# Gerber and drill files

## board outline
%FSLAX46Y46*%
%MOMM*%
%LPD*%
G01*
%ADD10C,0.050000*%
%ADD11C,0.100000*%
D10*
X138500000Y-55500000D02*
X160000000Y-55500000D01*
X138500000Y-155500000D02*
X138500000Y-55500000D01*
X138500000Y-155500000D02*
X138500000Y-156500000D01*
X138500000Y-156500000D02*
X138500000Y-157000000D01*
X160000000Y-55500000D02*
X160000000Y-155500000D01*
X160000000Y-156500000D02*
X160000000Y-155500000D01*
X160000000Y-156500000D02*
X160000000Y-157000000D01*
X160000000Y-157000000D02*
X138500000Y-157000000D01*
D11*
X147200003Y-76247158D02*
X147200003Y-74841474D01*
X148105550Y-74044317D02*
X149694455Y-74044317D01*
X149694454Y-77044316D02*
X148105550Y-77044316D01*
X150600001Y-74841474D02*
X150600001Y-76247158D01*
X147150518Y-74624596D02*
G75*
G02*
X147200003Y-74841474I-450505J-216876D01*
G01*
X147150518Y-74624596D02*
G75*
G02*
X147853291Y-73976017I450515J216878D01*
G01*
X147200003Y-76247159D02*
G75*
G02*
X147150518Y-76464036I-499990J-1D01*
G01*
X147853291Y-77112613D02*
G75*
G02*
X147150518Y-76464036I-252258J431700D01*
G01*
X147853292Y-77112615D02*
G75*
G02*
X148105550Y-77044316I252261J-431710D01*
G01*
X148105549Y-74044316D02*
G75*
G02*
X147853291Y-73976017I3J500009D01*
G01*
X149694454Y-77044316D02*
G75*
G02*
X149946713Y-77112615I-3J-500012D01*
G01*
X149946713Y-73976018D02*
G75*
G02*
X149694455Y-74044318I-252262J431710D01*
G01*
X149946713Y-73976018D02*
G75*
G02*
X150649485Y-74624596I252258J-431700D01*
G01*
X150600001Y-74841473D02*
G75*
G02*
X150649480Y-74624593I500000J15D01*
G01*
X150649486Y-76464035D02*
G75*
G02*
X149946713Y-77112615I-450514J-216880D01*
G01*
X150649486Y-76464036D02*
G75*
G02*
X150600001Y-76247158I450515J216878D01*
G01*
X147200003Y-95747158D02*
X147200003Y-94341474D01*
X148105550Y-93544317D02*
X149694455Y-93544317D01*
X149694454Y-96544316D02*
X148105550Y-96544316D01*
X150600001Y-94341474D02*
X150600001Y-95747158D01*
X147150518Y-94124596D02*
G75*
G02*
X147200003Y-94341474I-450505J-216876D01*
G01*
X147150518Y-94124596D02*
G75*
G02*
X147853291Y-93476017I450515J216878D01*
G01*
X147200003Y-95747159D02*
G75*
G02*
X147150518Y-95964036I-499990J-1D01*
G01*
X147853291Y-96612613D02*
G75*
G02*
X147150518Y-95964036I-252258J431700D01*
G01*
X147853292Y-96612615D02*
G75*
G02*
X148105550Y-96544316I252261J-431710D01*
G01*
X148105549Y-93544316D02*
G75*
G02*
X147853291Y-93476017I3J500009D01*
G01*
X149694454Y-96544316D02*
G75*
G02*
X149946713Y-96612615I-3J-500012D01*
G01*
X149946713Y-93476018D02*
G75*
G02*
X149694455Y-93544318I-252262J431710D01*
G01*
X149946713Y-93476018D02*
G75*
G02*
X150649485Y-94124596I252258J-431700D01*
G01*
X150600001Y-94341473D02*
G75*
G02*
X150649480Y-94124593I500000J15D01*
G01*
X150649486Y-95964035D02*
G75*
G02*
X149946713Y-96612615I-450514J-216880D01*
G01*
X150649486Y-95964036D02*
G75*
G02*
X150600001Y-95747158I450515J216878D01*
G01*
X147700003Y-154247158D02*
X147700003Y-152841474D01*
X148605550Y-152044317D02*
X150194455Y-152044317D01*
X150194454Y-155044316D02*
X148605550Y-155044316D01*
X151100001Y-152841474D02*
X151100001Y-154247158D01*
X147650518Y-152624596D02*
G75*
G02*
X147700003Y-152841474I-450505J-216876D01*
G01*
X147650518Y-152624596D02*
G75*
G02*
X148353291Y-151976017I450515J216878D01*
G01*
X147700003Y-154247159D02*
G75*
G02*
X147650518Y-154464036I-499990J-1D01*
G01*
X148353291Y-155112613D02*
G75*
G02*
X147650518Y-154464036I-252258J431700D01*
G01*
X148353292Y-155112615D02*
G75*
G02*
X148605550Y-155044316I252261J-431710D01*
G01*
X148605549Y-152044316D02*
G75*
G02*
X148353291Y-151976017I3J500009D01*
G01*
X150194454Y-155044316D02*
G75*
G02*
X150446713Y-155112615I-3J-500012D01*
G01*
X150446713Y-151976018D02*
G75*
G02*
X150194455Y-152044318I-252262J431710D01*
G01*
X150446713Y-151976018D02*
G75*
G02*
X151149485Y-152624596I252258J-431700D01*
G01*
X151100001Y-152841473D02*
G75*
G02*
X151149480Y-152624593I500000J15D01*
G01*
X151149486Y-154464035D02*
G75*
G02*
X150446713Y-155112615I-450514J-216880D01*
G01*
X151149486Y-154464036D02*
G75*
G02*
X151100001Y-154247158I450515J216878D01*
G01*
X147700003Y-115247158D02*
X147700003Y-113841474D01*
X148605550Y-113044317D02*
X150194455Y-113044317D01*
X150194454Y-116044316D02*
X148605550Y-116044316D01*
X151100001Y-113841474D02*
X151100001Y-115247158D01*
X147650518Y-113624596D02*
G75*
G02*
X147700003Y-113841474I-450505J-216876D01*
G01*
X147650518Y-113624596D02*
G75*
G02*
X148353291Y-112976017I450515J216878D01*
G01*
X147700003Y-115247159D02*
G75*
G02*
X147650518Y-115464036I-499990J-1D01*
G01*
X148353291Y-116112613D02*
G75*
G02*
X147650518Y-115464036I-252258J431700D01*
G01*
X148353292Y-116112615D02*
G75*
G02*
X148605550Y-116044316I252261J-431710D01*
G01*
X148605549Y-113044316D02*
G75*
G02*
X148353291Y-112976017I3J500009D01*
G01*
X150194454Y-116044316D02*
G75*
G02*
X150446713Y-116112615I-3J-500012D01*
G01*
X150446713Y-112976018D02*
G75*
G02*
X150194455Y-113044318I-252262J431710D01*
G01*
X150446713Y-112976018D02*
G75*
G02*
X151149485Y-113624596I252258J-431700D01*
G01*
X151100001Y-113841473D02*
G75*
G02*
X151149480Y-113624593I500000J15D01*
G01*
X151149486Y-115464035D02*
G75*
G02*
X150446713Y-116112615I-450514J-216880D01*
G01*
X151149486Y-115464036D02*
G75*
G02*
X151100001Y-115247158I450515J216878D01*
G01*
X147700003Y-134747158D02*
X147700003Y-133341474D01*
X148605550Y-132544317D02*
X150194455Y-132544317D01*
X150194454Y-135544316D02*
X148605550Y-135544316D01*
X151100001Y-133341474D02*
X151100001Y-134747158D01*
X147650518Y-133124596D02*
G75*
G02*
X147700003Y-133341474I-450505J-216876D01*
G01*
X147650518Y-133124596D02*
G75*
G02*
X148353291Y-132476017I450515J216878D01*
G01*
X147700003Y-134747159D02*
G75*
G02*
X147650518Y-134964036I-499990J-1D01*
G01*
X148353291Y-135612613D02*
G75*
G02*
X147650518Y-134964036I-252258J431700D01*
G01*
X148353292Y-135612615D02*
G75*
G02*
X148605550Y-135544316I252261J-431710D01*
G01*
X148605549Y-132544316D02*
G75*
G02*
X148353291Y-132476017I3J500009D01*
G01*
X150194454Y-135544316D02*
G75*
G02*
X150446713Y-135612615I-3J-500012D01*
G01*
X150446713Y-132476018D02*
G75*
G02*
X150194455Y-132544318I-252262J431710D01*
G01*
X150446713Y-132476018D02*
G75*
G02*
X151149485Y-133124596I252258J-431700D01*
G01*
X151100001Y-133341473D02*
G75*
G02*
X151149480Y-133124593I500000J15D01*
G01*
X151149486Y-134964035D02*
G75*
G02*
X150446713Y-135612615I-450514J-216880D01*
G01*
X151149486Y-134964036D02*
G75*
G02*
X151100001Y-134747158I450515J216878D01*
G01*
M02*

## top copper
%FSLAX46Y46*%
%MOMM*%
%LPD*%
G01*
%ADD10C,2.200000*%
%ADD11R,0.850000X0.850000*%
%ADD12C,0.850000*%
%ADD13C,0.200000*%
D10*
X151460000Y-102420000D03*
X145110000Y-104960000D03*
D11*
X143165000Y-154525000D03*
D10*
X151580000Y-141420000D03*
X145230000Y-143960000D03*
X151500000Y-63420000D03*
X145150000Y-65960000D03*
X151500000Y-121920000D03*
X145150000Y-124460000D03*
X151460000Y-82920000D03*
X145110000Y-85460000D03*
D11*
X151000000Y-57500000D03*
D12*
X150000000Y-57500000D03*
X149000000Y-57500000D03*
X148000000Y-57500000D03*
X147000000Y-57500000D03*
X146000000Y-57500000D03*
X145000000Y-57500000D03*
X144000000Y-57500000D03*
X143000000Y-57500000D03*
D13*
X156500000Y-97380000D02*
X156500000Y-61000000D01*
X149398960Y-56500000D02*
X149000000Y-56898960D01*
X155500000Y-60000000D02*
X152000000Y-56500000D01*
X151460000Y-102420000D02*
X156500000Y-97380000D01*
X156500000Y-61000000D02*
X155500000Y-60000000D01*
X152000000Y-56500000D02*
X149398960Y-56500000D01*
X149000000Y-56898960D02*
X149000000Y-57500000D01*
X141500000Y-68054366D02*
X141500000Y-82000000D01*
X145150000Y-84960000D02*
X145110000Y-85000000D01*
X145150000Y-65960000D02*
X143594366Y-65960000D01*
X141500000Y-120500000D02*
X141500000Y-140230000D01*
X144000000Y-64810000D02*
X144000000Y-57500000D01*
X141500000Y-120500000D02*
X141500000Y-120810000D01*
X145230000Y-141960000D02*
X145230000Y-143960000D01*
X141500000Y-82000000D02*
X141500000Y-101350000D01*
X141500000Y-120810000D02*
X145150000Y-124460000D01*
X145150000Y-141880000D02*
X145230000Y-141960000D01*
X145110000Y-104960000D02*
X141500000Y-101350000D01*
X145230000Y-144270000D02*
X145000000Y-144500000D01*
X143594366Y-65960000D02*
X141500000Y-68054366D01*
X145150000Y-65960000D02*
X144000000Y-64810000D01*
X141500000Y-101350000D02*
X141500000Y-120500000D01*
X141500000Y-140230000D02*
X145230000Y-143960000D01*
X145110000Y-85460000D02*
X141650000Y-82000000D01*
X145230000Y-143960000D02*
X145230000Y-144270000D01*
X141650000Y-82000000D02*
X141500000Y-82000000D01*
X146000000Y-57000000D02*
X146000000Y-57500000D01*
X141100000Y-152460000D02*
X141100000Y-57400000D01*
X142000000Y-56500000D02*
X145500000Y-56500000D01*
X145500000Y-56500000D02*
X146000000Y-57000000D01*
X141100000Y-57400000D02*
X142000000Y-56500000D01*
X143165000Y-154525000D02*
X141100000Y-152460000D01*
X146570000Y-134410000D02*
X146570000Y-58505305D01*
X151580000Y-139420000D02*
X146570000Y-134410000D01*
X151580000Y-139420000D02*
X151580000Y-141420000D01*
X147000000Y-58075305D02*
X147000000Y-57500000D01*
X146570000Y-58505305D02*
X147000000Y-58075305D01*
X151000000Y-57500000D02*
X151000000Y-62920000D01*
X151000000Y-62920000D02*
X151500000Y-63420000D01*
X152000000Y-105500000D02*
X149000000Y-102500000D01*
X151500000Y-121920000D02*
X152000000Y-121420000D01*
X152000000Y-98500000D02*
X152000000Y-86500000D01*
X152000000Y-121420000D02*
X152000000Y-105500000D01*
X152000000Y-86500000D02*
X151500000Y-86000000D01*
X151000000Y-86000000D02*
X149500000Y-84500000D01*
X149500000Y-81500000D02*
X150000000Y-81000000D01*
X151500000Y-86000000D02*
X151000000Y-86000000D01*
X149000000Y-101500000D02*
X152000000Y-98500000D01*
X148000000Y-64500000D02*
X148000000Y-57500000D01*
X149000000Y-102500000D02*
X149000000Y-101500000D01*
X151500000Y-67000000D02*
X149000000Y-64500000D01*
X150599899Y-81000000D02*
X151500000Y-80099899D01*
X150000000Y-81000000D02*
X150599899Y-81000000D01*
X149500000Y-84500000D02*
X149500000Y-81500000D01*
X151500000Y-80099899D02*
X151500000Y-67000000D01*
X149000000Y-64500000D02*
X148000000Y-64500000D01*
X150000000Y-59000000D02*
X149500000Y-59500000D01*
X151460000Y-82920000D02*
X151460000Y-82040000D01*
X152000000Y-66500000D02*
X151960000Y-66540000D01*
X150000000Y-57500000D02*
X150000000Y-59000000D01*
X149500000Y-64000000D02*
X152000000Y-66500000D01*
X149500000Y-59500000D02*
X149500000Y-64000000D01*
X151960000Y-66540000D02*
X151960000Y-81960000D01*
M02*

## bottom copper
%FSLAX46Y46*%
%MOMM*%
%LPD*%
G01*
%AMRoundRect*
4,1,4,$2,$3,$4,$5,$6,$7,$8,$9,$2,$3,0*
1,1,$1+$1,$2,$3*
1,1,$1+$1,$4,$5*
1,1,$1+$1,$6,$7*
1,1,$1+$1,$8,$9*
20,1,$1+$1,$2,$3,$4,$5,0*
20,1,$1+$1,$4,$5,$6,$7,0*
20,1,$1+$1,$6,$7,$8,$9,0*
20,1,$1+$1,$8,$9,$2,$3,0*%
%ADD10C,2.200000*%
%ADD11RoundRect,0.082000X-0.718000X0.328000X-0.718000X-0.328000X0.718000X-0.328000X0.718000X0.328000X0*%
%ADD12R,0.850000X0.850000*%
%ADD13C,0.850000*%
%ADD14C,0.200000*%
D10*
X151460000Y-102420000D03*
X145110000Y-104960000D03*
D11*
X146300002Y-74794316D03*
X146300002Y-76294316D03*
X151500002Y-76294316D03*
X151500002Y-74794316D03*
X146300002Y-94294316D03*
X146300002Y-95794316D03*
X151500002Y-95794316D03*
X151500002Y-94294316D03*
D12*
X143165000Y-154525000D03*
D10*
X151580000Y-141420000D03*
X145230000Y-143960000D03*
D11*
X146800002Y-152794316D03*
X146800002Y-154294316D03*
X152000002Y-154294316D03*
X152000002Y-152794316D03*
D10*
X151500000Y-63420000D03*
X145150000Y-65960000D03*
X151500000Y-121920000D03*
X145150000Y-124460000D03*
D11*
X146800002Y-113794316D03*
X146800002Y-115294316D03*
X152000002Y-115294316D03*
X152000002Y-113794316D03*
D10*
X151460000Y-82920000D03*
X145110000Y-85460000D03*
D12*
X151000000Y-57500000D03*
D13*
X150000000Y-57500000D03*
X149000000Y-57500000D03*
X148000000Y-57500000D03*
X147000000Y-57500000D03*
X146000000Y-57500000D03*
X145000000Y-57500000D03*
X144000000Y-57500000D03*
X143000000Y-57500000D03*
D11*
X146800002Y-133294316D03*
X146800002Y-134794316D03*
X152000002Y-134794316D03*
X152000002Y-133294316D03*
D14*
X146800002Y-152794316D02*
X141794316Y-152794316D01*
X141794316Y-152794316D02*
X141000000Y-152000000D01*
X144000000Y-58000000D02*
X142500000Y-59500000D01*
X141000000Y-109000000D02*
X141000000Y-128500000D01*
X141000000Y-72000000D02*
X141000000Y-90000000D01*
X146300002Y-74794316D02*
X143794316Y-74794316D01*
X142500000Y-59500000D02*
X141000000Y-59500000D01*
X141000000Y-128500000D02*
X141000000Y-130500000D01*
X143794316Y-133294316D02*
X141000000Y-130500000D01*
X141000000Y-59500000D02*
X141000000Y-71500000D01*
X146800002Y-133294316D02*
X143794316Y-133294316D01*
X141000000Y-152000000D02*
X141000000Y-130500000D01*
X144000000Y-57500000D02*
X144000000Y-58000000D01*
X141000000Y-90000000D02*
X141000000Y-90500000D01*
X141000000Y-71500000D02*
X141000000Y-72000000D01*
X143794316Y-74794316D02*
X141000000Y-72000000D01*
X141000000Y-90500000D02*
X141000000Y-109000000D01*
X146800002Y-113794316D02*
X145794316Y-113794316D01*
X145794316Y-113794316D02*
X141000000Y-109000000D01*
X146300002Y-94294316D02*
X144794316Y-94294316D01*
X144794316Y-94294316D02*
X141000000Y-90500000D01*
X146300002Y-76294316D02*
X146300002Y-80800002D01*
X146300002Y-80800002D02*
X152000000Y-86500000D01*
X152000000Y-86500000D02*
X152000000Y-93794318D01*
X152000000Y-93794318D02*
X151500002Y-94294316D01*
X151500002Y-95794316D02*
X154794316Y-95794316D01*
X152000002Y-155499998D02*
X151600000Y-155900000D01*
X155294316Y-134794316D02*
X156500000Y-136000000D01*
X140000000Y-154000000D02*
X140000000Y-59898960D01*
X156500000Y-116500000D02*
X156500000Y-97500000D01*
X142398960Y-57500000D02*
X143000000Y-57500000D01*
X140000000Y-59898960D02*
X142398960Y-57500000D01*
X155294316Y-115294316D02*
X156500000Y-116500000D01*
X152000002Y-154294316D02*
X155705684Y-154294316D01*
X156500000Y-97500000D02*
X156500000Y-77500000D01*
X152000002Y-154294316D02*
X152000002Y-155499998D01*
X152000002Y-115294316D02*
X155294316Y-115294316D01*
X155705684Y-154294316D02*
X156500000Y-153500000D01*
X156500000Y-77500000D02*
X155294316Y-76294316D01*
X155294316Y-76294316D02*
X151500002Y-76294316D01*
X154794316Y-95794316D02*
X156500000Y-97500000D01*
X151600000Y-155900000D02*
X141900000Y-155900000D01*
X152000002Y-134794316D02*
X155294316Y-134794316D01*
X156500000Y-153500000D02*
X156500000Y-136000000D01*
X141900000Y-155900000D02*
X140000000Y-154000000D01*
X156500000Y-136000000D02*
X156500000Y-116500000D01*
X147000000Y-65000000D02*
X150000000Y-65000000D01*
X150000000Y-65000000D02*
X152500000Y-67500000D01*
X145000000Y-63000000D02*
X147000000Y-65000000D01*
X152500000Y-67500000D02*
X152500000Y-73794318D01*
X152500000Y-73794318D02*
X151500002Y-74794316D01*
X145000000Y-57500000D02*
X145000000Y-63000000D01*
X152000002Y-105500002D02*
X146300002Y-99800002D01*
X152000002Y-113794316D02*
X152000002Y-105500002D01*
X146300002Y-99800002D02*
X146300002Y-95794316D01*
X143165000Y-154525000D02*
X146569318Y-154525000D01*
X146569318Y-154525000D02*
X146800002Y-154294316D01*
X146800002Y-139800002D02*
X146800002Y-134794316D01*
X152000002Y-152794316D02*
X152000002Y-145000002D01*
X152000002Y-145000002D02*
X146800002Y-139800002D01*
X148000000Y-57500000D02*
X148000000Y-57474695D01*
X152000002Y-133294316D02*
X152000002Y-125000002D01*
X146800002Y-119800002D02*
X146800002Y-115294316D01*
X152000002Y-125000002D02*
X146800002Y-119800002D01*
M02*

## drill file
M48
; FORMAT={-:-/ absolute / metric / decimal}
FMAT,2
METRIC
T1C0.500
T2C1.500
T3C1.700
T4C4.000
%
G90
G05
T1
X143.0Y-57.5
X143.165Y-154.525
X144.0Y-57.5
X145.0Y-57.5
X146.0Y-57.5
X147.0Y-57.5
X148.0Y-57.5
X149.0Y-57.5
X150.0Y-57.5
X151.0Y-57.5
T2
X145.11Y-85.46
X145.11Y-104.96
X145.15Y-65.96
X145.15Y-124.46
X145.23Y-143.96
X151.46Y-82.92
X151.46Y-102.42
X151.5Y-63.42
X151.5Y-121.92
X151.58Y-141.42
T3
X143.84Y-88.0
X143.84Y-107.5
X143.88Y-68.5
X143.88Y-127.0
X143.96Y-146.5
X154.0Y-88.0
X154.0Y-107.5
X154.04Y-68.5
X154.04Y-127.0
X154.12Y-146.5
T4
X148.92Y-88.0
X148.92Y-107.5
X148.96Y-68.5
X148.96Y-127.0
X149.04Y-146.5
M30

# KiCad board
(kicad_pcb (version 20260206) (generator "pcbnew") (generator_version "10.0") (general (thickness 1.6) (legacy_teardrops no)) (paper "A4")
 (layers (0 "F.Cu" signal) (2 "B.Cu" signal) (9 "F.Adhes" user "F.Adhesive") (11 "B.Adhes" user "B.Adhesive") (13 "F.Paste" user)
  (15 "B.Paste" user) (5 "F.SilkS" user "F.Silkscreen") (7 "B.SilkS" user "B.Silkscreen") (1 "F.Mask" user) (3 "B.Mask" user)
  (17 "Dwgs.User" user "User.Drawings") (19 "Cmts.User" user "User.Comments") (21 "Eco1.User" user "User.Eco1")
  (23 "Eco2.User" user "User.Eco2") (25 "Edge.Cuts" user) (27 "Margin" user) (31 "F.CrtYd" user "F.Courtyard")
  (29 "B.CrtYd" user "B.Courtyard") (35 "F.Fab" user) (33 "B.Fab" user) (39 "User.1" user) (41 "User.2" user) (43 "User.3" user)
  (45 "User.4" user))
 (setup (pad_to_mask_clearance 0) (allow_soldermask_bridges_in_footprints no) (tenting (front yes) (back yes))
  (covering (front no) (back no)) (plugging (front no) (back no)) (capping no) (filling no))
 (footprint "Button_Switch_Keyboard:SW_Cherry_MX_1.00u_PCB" (layer "F.Cu") (at 151.46 102.42)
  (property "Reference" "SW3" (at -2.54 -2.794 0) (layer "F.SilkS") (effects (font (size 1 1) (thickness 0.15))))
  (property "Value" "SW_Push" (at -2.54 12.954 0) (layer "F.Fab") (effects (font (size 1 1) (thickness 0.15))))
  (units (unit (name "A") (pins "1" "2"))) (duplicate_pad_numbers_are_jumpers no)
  (pad "" np_thru_hole circle (at -7.62 5.08) (size 1.7 1.7) (drill 1.7) (layers "*.Cu" "*.Mask"))
  (pad "" np_thru_hole circle (at -2.54 5.08) (size 4 4) (drill 4) (layers "*.Cu" "*.Mask"))
  (pad "" np_thru_hole circle (at 2.54 5.08) (size 1.7 1.7) (drill 1.7) (layers "*.Cu" "*.Mask"))
  (pad "1" thru_hole circle (at 0 0) (size 2.2 2.2) (drill 1.5) (layers "*.Cu" "*.Mask") (remove_unused_layers no) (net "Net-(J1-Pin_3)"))
  (pad "2" thru_hole circle (at -6.35 2.54) (size 2.2 2.2) (drill 1.5) (layers "*.Cu" "*.Mask") (remove_unused_layers no) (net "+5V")))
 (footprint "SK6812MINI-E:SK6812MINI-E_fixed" (layer "F.Cu") (at 148.900001 75.647158)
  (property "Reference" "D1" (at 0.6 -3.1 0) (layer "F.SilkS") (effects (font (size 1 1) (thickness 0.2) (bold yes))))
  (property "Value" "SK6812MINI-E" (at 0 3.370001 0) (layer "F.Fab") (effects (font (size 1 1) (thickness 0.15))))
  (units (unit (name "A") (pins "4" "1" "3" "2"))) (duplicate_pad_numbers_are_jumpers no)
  (fp_line (start -1.699998 0.6) (end -1.699998 -0.805684) (stroke (width 0.1) (type solid)) (layer "Edge.Cuts"))
  (fp_line (start -0.794451 -1.602841) (end 0.794454 -1.602841) (stroke (width 0.1) (type solid)) (layer "Edge.Cuts"))
  (fp_line (start 0.794453 1.397158) (end -0.794451 1.397158) (stroke (width 0.1) (type solid)) (layer "Edge.Cuts"))
  (fp_line (start 1.7 -0.805684) (end 1.7 0.6) (stroke (width 0.1) (type solid)) (layer "Edge.Cuts"))
  (fp_arc (start -1.749483 -1.022562) (mid -1.712526 -0.91691) (end -1.699998 -0.805684) (stroke (width 0.1) (type solid))
   (layer "Edge.Cuts"))
  (fp_arc (start -1.749483 -1.022562) (mid -1.63807 -1.606877) (end -1.04671 -1.671141) (stroke (width 0.1) (type solid))
   (layer "Edge.Cuts"))
  (fp_arc (start -1.699998 0.600001) (mid -1.712526 0.711226) (end -1.749483 0.816878) (stroke (width 0.1) (type solid)) (layer "Edge.Cuts"))
  (fp_arc (start -1.04671 1.465455) (mid -1.638069 1.401192) (end -1.749483 0.816878) (stroke (width 0.1) (type solid)) (layer "Edge.Cuts"))
  (fp_arc (start -1.046709 1.465457) (mid -0.925121 1.414535) (end -0.794451 1.397158) (stroke (width 0.1) (type solid)) (layer "Edge.Cuts"))
  (fp_arc (start -0.794452 -1.602842) (mid -0.925122 -1.620219) (end -1.04671 -1.671141) (stroke (width 0.1) (type solid))
   (layer "Edge.Cuts"))
  (fp_arc (start 0.794453 1.397158) (mid 0.925124 1.414535) (end 1.046712 1.465457) (stroke (width 0.1) (type solid)) (layer "Edge.Cuts"))
  (fp_arc (start 1.046712 -1.67114) (mid 0.925124 -1.620218) (end 0.794454 -1.602841) (stroke (width 0.1) (type solid)) (layer "Edge.Cuts"))
  (fp_arc (start 1.046712 -1.67114) (mid 1.638072 -1.606876) (end 1.749485 -1.022562) (stroke (width 0.1) (type solid)) (layer "Edge.Cuts"))
  (fp_arc (start 1.7 -0.805685) (mid 1.712528 -0.91691) (end 1.749485 -1.022562) (stroke (width 0.1) (type solid)) (layer "Edge.Cuts"))
  (fp_arc (start 1.749485 0.816877) (mid 1.638073 1.401193) (end 1.046712 1.465457) (stroke (width 0.1) (type solid)) (layer "Edge.Cuts"))
  (fp_arc (start 1.749485 0.816878) (mid 1.712528 0.711226) (end 1.7 0.6) (stroke (width 0.1) (type solid)) (layer "Edge.Cuts"))
  (pad "1" smd roundrect (at -2.599999 -0.852842 270) (size 0.82 1.6) (layers "B.Cu" "B.Mask" "B.Paste") (roundrect_rratio 0.1) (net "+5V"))
  (pad "2" smd roundrect (at -2.599999 0.647158 270) (size 0.82 1.6) (layers "B.Cu" "B.Mask" "B.Paste") (roundrect_rratio 0.1)
   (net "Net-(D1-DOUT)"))
  (pad "3" smd roundrect (at 2.600001 0.647158 270) (size 0.82 1.6) (layers "B.Cu" "B.Mask" "B.Paste") (roundrect_rratio 0.1) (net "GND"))
  (pad "4" smd roundrect (at 2.600001 -0.852842 270) (size 0.82 1.6) (layers "B.Cu" "B.Mask" "B.Paste") (roundrect_rratio 0.1)
   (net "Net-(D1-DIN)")))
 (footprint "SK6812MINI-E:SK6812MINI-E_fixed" (layer "F.Cu") (at 148.900001 95.147158)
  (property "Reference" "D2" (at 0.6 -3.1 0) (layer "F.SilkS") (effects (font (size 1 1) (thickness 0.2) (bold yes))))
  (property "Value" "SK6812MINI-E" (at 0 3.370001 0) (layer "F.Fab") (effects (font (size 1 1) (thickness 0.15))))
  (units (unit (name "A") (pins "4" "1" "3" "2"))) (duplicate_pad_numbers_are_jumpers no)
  (fp_line (start -1.699998 0.6) (end -1.699998 -0.805684) (stroke (width 0.1) (type solid)) (layer "Edge.Cuts"))
  (fp_line (start -0.794451 -1.602841) (end 0.794454 -1.602841) (stroke (width 0.1) (type solid)) (layer "Edge.Cuts"))
  (fp_line (start 0.794453 1.397158) (end -0.794451 1.397158) (stroke (width 0.1) (type solid)) (layer "Edge.Cuts"))
  (fp_line (start 1.7 -0.805684) (end 1.7 0.6) (stroke (width 0.1) (type solid)) (layer "Edge.Cuts"))
  (fp_arc (start -1.749483 -1.022562) (mid -1.712526 -0.91691) (end -1.699998 -0.805684) (stroke (width 0.1) (type solid))
   (layer "Edge.Cuts"))
  (fp_arc (start -1.749483 -1.022562) (mid -1.63807 -1.606877) (end -1.04671 -1.671141) (stroke (width 0.1) (type solid))
   (layer "Edge.Cuts"))
  (fp_arc (start -1.699998 0.600001) (mid -1.712526 0.711226) (end -1.749483 0.816878) (stroke (width 0.1) (type solid)) (layer "Edge.Cuts"))
  (fp_arc (start -1.04671 1.465455) (mid -1.638069 1.401192) (end -1.749483 0.816878) (stroke (width 0.1) (type solid)) (layer "Edge.Cuts"))
  (fp_arc (start -1.046709 1.465457) (mid -0.925121 1.414535) (end -0.794451 1.397158) (stroke (width 0.1) (type solid)) (layer "Edge.Cuts"))
  (fp_arc (start -0.794452 -1.602842) (mid -0.925122 -1.620219) (end -1.04671 -1.671141) (stroke (width 0.1) (type solid))
   (layer "Edge.Cuts"))
  (fp_arc (start 0.794453 1.397158) (mid 0.925124 1.414535) (end 1.046712 1.465457) (stroke (width 0.1) (type solid)) (layer "Edge.Cuts"))
  (fp_arc (start 1.046712 -1.67114) (mid 0.925124 -1.620218) (end 0.794454 -1.602841) (stroke (width 0.1) (type solid)) (layer "Edge.Cuts"))
  (fp_arc (start 1.046712 -1.67114) (mid 1.638072 -1.606876) (end 1.749485 -1.022562) (stroke (width 0.1) (type solid)) (layer "Edge.Cuts"))
  (fp_arc (start 1.7 -0.805685) (mid 1.712528 -0.91691) (end 1.749485 -1.022562) (stroke (width 0.1) (type solid)) (layer "Edge.Cuts"))
  (fp_arc (start 1.749485 0.816877) (mid 1.638073 1.401193) (end 1.046712 1.465457) (stroke (width 0.1) (type solid)) (layer "Edge.Cuts"))
  (fp_arc (start 1.749485 0.816878) (mid 1.712528 0.711226) (end 1.7 0.6) (stroke (width 0.1) (type solid)) (layer "Edge.Cuts"))
  (pad "1" smd roundrect (at -2.599999 -0.852842 270) (size 0.82 1.6) (layers "B.Cu" "B.Mask" "B.Paste") (roundrect_rratio 0.1) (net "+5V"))
  (pad "2" smd roundrect (at -2.599999 0.647158 270) (size 0.82 1.6) (layers "B.Cu" "B.Mask" "B.Paste") (roundrect_rratio 0.1)
   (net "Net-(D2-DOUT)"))
  (pad "3" smd roundrect (at 2.600001 0.647158 270) (size 0.82 1.6) (layers "B.Cu" "B.Mask" "B.Paste") (roundrect_rratio 0.1) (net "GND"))
  (pad "4" smd roundrect (at 2.600001 -0.852842 270) (size 0.82 1.6) (layers "B.Cu" "B.Mask" "B.Paste") (roundrect_rratio 0.1)
   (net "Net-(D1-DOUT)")))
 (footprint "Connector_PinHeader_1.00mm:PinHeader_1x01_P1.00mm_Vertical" (layer "F.Cu") (at 143.165 154.525)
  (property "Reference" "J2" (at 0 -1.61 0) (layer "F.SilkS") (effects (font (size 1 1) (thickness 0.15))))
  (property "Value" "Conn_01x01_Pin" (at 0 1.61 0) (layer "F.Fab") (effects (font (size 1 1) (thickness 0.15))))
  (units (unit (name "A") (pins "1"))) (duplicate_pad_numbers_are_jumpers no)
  (pad "1" thru_hole rect (at 0 0) (size 0.85 0.85) (drill 0.5) (layers "*.Cu" "*.Mask") (remove_unused_layers no) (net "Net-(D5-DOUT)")))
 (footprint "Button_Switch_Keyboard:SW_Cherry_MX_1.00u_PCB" (layer "F.Cu") (at 151.58 141.42)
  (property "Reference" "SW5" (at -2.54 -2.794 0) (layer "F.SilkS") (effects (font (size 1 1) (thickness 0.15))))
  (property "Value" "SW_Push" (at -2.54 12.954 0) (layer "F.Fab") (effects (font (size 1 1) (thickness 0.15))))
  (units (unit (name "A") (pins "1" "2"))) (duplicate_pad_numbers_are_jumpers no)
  (pad "" np_thru_hole circle (at -7.62 5.08) (size 1.7 1.7) (drill 1.7) (layers "*.Cu" "*.Mask"))
  (pad "" np_thru_hole circle (at -2.54 5.08) (size 4 4) (drill 4) (layers "*.Cu" "*.Mask"))
  (pad "" np_thru_hole circle (at 2.54 5.08) (size 1.7 1.7) (drill 1.7) (layers "*.Cu" "*.Mask"))
  (pad "1" thru_hole circle (at 0 0) (size 2.2 2.2) (drill 1.5) (layers "*.Cu" "*.Mask") (remove_unused_layers no) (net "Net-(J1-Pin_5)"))
  (pad "2" thru_hole circle (at -6.35 2.54) (size 2.2 2.2) (drill 1.5) (layers "*.Cu" "*.Mask") (remove_unused_layers no) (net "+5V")))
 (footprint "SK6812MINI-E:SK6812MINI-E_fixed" (layer "F.Cu") (at 149.400001 153.647158)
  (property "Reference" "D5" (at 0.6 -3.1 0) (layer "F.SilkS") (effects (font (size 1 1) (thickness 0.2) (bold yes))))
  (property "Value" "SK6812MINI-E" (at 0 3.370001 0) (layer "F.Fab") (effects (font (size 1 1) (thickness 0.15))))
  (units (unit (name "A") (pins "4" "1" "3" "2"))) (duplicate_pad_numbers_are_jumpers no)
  (fp_line (start -1.699998 0.6) (end -1.699998 -0.805684) (stroke (width 0.1) (type solid)) (layer "Edge.Cuts"))
  (fp_line (start -0.794451 -1.602841) (end 0.794454 -1.602841) (stroke (width 0.1) (type solid)) (layer "Edge.Cuts"))
  (fp_line (start 0.794453 1.397158) (end -0.794451 1.397158) (stroke (width 0.1) (type solid)) (layer "Edge.Cuts"))
  (fp_line (start 1.7 -0.805684) (end 1.7 0.6) (stroke (width 0.1) (type solid)) (layer "Edge.Cuts"))
  (fp_arc (start -1.749483 -1.022562) (mid -1.712526 -0.91691) (end -1.699998 -0.805684) (stroke (width 0.1) (type solid))
   (layer "Edge.Cuts"))
  (fp_arc (start -1.749483 -1.022562) (mid -1.63807 -1.606877) (end -1.04671 -1.671141) (stroke (width 0.1) (type solid))
   (layer "Edge.Cuts"))
  (fp_arc (start -1.699998 0.600001) (mid -1.712526 0.711226) (end -1.749483 0.816878) (stroke (width 0.1) (type solid)) (layer "Edge.Cuts"))
  (fp_arc (start -1.04671 1.465455) (mid -1.638069 1.401192) (end -1.749483 0.816878) (stroke (width 0.1) (type solid)) (layer "Edge.Cuts"))
  (fp_arc (start -1.046709 1.465457) (mid -0.925121 1.414535) (end -0.794451 1.397158) (stroke (width 0.1) (type solid)) (layer "Edge.Cuts"))
  (fp_arc (start -0.794452 -1.602842) (mid -0.925122 -1.620219) (end -1.04671 -1.671141) (stroke (width 0.1) (type solid))
   (layer "Edge.Cuts"))
  (fp_arc (start 0.794453 1.397158) (mid 0.925124 1.414535) (end 1.046712 1.465457) (stroke (width 0.1) (type solid)) (layer "Edge.Cuts"))
  (fp_arc (start 1.046712 -1.67114) (mid 0.925124 -1.620218) (end 0.794454 -1.602841) (stroke (width 0.1) (type solid)) (layer "Edge.Cuts"))
  (fp_arc (start 1.046712 -1.67114) (mid 1.638072 -1.606876) (end 1.749485 -1.022562) (stroke (width 0.1) (type solid)) (layer "Edge.Cuts"))
  (fp_arc (start 1.7 -0.805685) (mid 1.712528 -0.91691) (end 1.749485 -1.022562) (stroke (width 0.1) (type solid)) (layer "Edge.Cuts"))
  (fp_arc (start 1.749485 0.816877) (mid 1.638073 1.401193) (end 1.046712 1.465457) (stroke (width 0.1) (type solid)) (layer "Edge.Cuts"))
  (fp_arc (start 1.749485 0.816878) (mid 1.712528 0.711226) (end 1.7 0.6) (stroke (width 0.1) (type solid)) (layer "Edge.Cuts"))
  (pad "1" smd roundrect (at -2.599999 -0.852842 270) (size 0.82 1.6) (layers "B.Cu" "B.Mask" "B.Paste") (roundrect_rratio 0.1) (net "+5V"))
  (pad "2" smd roundrect (at -2.599999 0.647158 270) (size 0.82 1.6) (layers "B.Cu" "B.Mask" "B.Paste") (roundrect_rratio 0.1)
   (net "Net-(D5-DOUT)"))
  (pad "3" smd roundrect (at 2.600001 0.647158 270) (size 0.82 1.6) (layers "B.Cu" "B.Mask" "B.Paste") (roundrect_rratio 0.1) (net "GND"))
  (pad "4" smd roundrect (at 2.600001 -0.852842 270) (size 0.82 1.6) (layers "B.Cu" "B.Mask" "B.Paste") (roundrect_rratio 0.1)
   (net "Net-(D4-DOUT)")))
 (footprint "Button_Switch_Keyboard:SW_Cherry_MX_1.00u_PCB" (layer "F.Cu") (at 151.5 63.42)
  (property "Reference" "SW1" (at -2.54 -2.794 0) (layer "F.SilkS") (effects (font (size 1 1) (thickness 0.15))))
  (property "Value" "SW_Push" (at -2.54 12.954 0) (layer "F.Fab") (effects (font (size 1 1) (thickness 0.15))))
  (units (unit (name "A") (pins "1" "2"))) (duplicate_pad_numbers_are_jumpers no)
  (pad "" np_thru_hole circle (at -7.62 5.08) (size 1.7 1.7) (drill 1.7) (layers "*.Cu" "*.Mask"))
  (pad "" np_thru_hole circle (at -2.54 5.08) (size 4 4) (drill 4) (layers "*.Cu" "*.Mask"))
  (pad "" np_thru_hole circle (at 2.54 5.08) (size 1.7 1.7) (drill 1.7) (layers "*.Cu" "*.Mask"))
  (pad "1" thru_hole circle (at 0 0) (size 2.2 2.2) (drill 1.5) (layers "*.Cu" "*.Mask") (remove_unused_layers no) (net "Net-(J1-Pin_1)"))
  (pad "2" thru_hole circle (at -6.35 2.54) (size 2.2 2.2) (drill 1.5) (layers "*.Cu" "*.Mask") (remove_unused_layers no) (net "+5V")))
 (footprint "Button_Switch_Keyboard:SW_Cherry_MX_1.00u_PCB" (layer "F.Cu") (at 151.5 121.92)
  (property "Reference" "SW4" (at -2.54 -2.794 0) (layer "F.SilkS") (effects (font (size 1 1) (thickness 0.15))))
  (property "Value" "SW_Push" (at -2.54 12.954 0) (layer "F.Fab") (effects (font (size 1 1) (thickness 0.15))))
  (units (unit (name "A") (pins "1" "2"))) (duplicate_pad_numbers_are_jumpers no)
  (pad "" np_thru_hole circle (at -7.62 5.08) (size 1.7 1.7) (drill 1.7) (layers "*.Cu" "*.Mask"))
  (pad "" np_thru_hole circle (at -2.54 5.08) (size 4 4) (drill 4) (layers "*.Cu" "*.Mask"))
  (pad "" np_thru_hole circle (at 2.54 5.08) (size 1.7 1.7) (drill 1.7) (layers "*.Cu" "*.Mask"))
  (pad "1" thru_hole circle (at 0 0) (size 2.2 2.2) (drill 1.5) (layers "*.Cu" "*.Mask") (remove_unused_layers no) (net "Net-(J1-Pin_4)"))
  (pad "2" thru_hole circle (at -6.35 2.54) (size 2.2 2.2) (drill 1.5) (layers "*.Cu" "*.Mask") (remove_unused_layers no) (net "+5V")))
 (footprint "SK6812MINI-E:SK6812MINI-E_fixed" (layer "F.Cu") (at 149.400001 114.647158)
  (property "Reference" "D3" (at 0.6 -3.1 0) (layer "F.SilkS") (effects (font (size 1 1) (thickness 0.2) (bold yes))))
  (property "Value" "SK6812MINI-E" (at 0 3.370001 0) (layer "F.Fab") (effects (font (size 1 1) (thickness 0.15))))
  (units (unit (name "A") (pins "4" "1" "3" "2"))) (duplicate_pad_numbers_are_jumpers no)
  (fp_line (start -1.699998 0.6) (end -1.699998 -0.805684) (stroke (width 0.1) (type solid)) (layer "Edge.Cuts"))
  (fp_line (start -0.794451 -1.602841) (end 0.794454 -1.602841) (stroke (width 0.1) (type solid)) (layer "Edge.Cuts"))
  (fp_line (start 0.794453 1.397158) (end -0.794451 1.397158) (stroke (width 0.1) (type solid)) (layer "Edge.Cuts"))
  (fp_line (start 1.7 -0.805684) (end 1.7 0.6) (stroke (width 0.1) (type solid)) (layer "Edge.Cuts"))
  (fp_arc (start -1.749483 -1.022562) (mid -1.712526 -0.91691) (end -1.699998 -0.805684) (stroke (width 0.1) (type solid))
   (layer "Edge.Cuts"))
  (fp_arc (start -1.749483 -1.022562) (mid -1.63807 -1.606877) (end -1.04671 -1.671141) (stroke (width 0.1) (type solid))
   (layer "Edge.Cuts"))
  (fp_arc (start -1.699998 0.600001) (mid -1.712526 0.711226) (end -1.749483 0.816878) (stroke (width 0.1) (type solid)) (layer "Edge.Cuts"))
  (fp_arc (start -1.04671 1.465455) (mid -1.638069 1.401192) (end -1.749483 0.816878) (stroke (width 0.1) (type solid)) (layer "Edge.Cuts"))
  (fp_arc (start -1.046709 1.465457) (mid -0.925121 1.414535) (end -0.794451 1.397158) (stroke (width 0.1) (type solid)) (layer "Edge.Cuts"))
  (fp_arc (start -0.794452 -1.602842) (mid -0.925122 -1.620219) (end -1.04671 -1.671141) (stroke (width 0.1) (type solid))
   (layer "Edge.Cuts"))
  (fp_arc (start 0.794453 1.397158) (mid 0.925124 1.414535) (end 1.046712 1.465457) (stroke (width 0.1) (type solid)) (layer "Edge.Cuts"))
  (fp_arc (start 1.046712 -1.67114) (mid 0.925124 -1.620218) (end 0.794454 -1.602841) (stroke (width 0.1) (type solid)) (layer "Edge.Cuts"))
  (fp_arc (start 1.046712 -1.67114) (mid 1.638072 -1.606876) (end 1.749485 -1.022562) (stroke (width 0.1) (type solid)) (layer "Edge.Cuts"))
  (fp_arc (start 1.7 -0.805685) (mid 1.712528 -0.91691) (end 1.749485 -1.022562) (stroke (width 0.1) (type solid)) (layer "Edge.Cuts"))
  (fp_arc (start 1.749485 0.816877) (mid 1.638073 1.401193) (end 1.046712 1.465457) (stroke (width 0.1) (type solid)) (layer "Edge.Cuts"))
  (fp_arc (start 1.749485 0.816878) (mid 1.712528 0.711226) (end 1.7 0.6) (stroke (width 0.1) (type solid)) (layer "Edge.Cuts"))
  (pad "1" smd roundrect (at -2.599999 -0.852842 270) (size 0.82 1.6) (layers "B.Cu" "B.Mask" "B.Paste") (roundrect_rratio 0.1) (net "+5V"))
  (pad "2" smd roundrect (at -2.599999 0.647158 270) (size 0.82 1.6) (layers "B.Cu" "B.Mask" "B.Paste") (roundrect_rratio 0.1)
   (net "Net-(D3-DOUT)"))
  (pad "3" smd roundrect (at 2.600001 0.647158 270) (size 0.82 1.6) (layers "B.Cu" "B.Mask" "B.Paste") (roundrect_rratio 0.1) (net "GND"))
  (pad "4" smd roundrect (at 2.600001 -0.852842 270) (size 0.82 1.6) (layers "B.Cu" "B.Mask" "B.Paste") (roundrect_rratio 0.1)
   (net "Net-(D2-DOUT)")))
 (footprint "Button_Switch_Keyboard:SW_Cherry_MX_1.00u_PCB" (layer "F.Cu") (at 151.46 82.92)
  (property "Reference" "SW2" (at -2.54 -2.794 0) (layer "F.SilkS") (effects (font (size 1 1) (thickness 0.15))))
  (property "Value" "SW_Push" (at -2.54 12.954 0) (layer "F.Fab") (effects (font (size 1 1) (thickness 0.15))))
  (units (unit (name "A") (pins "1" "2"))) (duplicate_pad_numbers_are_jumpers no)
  (pad "" np_thru_hole circle (at -7.62 5.08) (size 1.7 1.7) (drill 1.7) (layers "*.Cu" "*.Mask"))
  (pad "" np_thru_hole circle (at -2.54 5.08) (size 4 4) (drill 4) (layers "*.Cu" "*.Mask"))
  (pad "" np_thru_hole circle (at 2.54 5.08) (size 1.7 1.7) (drill 1.7) (layers "*.Cu" "*.Mask"))
  (pad "1" thru_hole circle (at 0 0) (size 2.2 2.2) (drill 1.5) (layers "*.Cu" "*.Mask") (remove_unused_layers no) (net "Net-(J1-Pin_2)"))
  (pad "2" thru_hole circle (at -6.35 2.54) (size 2.2 2.2) (drill 1.5) (layers "*.Cu" "*.Mask") (remove_unused_layers no) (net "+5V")))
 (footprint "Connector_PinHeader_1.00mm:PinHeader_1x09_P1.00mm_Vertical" (layer "F.Cu") (at 151 57.5 -90)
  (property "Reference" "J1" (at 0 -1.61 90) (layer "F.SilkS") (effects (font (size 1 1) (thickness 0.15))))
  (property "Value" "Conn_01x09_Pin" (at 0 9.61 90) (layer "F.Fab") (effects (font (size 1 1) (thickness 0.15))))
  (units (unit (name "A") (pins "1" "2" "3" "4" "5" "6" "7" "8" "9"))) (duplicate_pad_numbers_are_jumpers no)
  (pad "1" thru_hole rect (at 0 0 270) (size 0.85 0.85) (drill 0.5) (layers "*.Cu" "*.Mask") (remove_unused_layers no)
   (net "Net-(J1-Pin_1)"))
  (pad "2" thru_hole circle (at 0 1 270) (size 0.85 0.85) (drill 0.5) (layers "*.Cu" "*.Mask") (remove_unused_layers no)
   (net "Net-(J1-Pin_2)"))
  (pad "3" thru_hole circle (at 0 2 270) (size 0.85 0.85) (drill 0.5) (layers "*.Cu" "*.Mask") (remove_unused_layers no)
   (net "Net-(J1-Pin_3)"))
  (pad "4" thru_hole circle (at 0 3 270) (size 0.85 0.85) (drill 0.5) (layers "*.Cu" "*.Mask") (remove_unused_layers no)
   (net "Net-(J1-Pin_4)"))
  (pad "5" thru_hole circle (at 0 4 270) (size 0.85 0.85) (drill 0.5) (layers "*.Cu" "*.Mask") (remove_unused_layers no)
   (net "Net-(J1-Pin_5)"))
  (pad "6" thru_hole circle (at 0 5 270) (size 0.85 0.85) (drill 0.5) (layers "*.Cu" "*.Mask") (remove_unused_layers no)
   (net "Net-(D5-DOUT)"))
  (pad "7" thru_hole circle (at 0 6 270) (size 0.85 0.85) (drill 0.5) (layers "*.Cu" "*.Mask") (remove_unused_layers no)
   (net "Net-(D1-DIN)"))
  (pad "8" thru_hole circle (at 0 7 270) (size 0.85 0.85) (drill 0.5) (layers "*.Cu" "*.Mask") (remove_unused_layers no) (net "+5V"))
  (pad "9" thru_hole circle (at 0 8 270) (size 0.85 0.85) (drill 0.5) (layers "*.Cu" "*.Mask") (remove_unused_layers no) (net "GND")))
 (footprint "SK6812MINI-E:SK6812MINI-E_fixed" (layer "F.Cu") (at 149.400001 134.147158)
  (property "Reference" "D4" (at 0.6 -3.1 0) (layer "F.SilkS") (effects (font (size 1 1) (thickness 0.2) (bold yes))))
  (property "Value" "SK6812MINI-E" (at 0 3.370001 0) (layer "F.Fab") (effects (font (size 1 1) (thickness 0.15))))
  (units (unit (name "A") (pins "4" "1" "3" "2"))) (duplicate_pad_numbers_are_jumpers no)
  (fp_line (start -1.699998 0.6) (end -1.699998 -0.805684) (stroke (width 0.1) (type solid)) (layer "Edge.Cuts"))
  (fp_line (start -0.794451 -1.602841) (end 0.794454 -1.602841) (stroke (width 0.1) (type solid)) (layer "Edge.Cuts"))
  (fp_line (start 0.794453 1.397158) (end -0.794451 1.397158) (stroke (width 0.1) (type solid)) (layer "Edge.Cuts"))
  (fp_line (start 1.7 -0.805684) (end 1.7 0.6) (stroke (width 0.1) (type solid)) (layer "Edge.Cuts"))
  (fp_arc (start -1.749483 -1.022562) (mid -1.712526 -0.91691) (end -1.699998 -0.805684) (stroke (width 0.1) (type solid))
   (layer "Edge.Cuts"))
  (fp_arc (start -1.749483 -1.022562) (mid -1.63807 -1.606877) (end -1.04671 -1.671141) (stroke (width 0.1) (type solid))
   (layer "Edge.Cuts"))
  (fp_arc (start -1.699998 0.600001) (mid -1.712526 0.711226) (end -1.749483 0.816878) (stroke (width 0.1) (type solid)) (layer "Edge.Cuts"))
  (fp_arc (start -1.04671 1.465455) (mid -1.638069 1.401192) (end -1.749483 0.816878) (stroke (width 0.1) (type solid)) (layer "Edge.Cuts"))
  (fp_arc (start -1.046709 1.465457) (mid -0.925121 1.414535) (end -0.794451 1.397158) (stroke (width 0.1) (type solid)) (layer "Edge.Cuts"))
  (fp_arc (start -0.794452 -1.602842) (mid -0.925122 -1.620219) (end -1.04671 -1.671141) (stroke (width 0.1) (type solid))
   (layer "Edge.Cuts"))
  (fp_arc (start 0.794453 1.397158) (mid 0.925124 1.414535) (end 1.046712 1.465457) (stroke (width 0.1) (type solid)) (layer "Edge.Cuts"))
  (fp_arc (start 1.046712 -1.67114) (mid 0.925124 -1.620218) (end 0.794454 -1.602841) (stroke (width 0.1) (type solid)) (layer "Edge.Cuts"))
  (fp_arc (start 1.046712 -1.67114) (mid 1.638072 -1.606876) (end 1.749485 -1.022562) (stroke (width 0.1) (type solid)) (layer "Edge.Cuts"))
  (fp_arc (start 1.7 -0.805685) (mid 1.712528 -0.91691) (end 1.749485 -1.022562) (stroke (width 0.1) (type solid)) (layer "Edge.Cuts"))
  (fp_arc (start 1.749485 0.816877) (mid 1.638073 1.401193) (end 1.046712 1.465457) (stroke (width 0.1) (type solid)) (layer "Edge.Cuts"))
  (fp_arc (start 1.749485 0.816878) (mid 1.712528 0.711226) (end 1.7 0.6) (stroke (width 0.1) (type solid)) (layer "Edge.Cuts"))
  (pad "1" smd roundrect (at -2.599999 -0.852842 270) (size 0.82 1.6) (layers "B.Cu" "B.Mask" "B.Paste") (roundrect_rratio 0.1) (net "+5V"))
  (pad "2" smd roundrect (at -2.599999 0.647158 270) (size 0.82 1.6) (layers "B.Cu" "B.Mask" "B.Paste") (roundrect_rratio 0.1)
   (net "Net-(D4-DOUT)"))
  (pad "3" smd roundrect (at 2.600001 0.647158 270) (size 0.82 1.6) (layers "B.Cu" "B.Mask" "B.Paste") (roundrect_rratio 0.1) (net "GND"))
  (pad "4" smd roundrect (at 2.600001 -0.852842 270) (size 0.82 1.6) (layers "B.Cu" "B.Mask" "B.Paste") (roundrect_rratio 0.1)
   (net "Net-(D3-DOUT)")))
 (gr_line (start 138.5 55.5) (end 160 55.5) (stroke (width 0.05) (type default)) (layer "Edge.Cuts"))
 (gr_line (start 138.5 155.5) (end 138.5 55.5) (stroke (width 0.05) (type default)) (layer "Edge.Cuts"))
 (gr_line (start 138.5 155.5) (end 138.5 156.5) (stroke (width 0.05) (type default)) (layer "Edge.Cuts"))
 (gr_line (start 138.5 156.5) (end 138.5 157) (stroke (width 0.05) (type default)) (layer "Edge.Cuts"))
 (gr_line (start 160 55.5) (end 160 155.5) (stroke (width 0.05) (type default)) (layer "Edge.Cuts"))
 (gr_line (start 160 156.5) (end 160 155.5) (stroke (width 0.05) (type default)) (layer "Edge.Cuts"))
 (gr_line (start 160 156.5) (end 160 157) (stroke (width 0.05) (type default)) (layer "Edge.Cuts"))
 (gr_line (start 160 157) (end 138.5 157) (stroke (width 0.05) (type default)) (layer "Edge.Cuts"))
 (segment (start 156.5 97.38) (end 156.5 61) (width 0.2) (layer "F.Cu") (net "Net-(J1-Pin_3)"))
 (segment (start 149.39896 56.5) (end 149 56.89896) (width 0.2) (layer "F.Cu") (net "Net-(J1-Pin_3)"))
 (segment (start 155.5 60) (end 152 56.5) (width 0.2) (layer "F.Cu") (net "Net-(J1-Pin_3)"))
 (segment (start 151.46 102.42) (end 156.5 97.38) (width 0.2) (layer "F.Cu") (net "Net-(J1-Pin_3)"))
 (segment (start 156.5 61) (end 155.5 60) (width 0.2) (layer "F.Cu") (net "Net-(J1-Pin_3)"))
 (segment (start 152 56.5) (end 149.39896 56.5) (width 0.2) (layer "F.Cu") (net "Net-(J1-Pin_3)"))
 (segment (start 149 56.89896) (end 149 57.5) (width 0.2) (layer "F.Cu") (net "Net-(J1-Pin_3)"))
 (segment (start 141.5 68.054366) (end 141.5 82) (width 0.2) (layer "F.Cu") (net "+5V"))
 (segment (start 145.15 84.96) (end 145.11 85) (width 0.2) (layer "F.Cu") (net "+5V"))
 (segment (start 145.15 65.96) (end 143.594366 65.96) (width 0.2) (layer "F.Cu") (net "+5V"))
 (segment (start 141.5 120.5) (end 141.5 140.23) (width 0.2) (layer "F.Cu") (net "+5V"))
 (segment (start 144 64.81) (end 144 57.5) (width 0.2) (layer "F.Cu") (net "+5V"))
 (segment (start 141.5 120.5) (end 141.5 120.81) (width 0.2) (layer "F.Cu") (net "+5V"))
 (segment (start 145.23 141.96) (end 145.23 143.96) (width 0.2) (layer "F.Cu") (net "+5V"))
 (segment (start 141.5 82) (end 141.5 101.35) (width 0.2) (layer "F.Cu") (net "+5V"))
 (segment (start 141.5 120.81) (end 145.15 124.46) (width 0.2) (layer "F.Cu") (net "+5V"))
 (segment (start 145.15 141.88) (end 145.23 141.96) (width 0.2) (layer "F.Cu") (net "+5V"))
 (segment (start 145.11 104.96) (end 141.5 101.35) (width 0.2) (layer "F.Cu") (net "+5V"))
 (segment (start 145.23 144.27) (end 145 144.5) (width 0.2) (layer "F.Cu") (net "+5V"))
 (segment (start 143.594366 65.96) (end 141.5 68.054366) (width 0.2) (layer "F.Cu") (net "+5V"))
 (segment (start 145.15 65.96) (end 144 64.81) (width 0.2) (layer "F.Cu") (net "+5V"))
 (segment (start 141.5 101.35) (end 141.5 120.5) (width 0.2) (layer "F.Cu") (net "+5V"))
 (segment (start 141.5 140.23) (end 145.23 143.96) (width 0.2) (layer "F.Cu") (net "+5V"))
 (segment (start 145.11 85.46) (end 141.65 82) (width 0.2) (layer "F.Cu") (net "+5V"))
 (segment (start 145.23 143.96) (end 145.23 144.27) (width 0.2) (layer "F.Cu") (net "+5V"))
 (segment (start 141.65 82) (end 141.5 82) (width 0.2) (layer "F.Cu") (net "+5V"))
 (segment (start 146.800002 152.794316) (end 141.794316 152.794316) (width 0.2) (layer "B.Cu") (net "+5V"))
 (segment (start 141.794316 152.794316) (end 141 152) (width 0.2) (layer "B.Cu") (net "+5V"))
 (segment (start 144 58) (end 142.5 59.5) (width 0.2) (layer "B.Cu") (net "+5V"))
 (segment (start 141 109) (end 141 128.5) (width 0.2) (layer "B.Cu") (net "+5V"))
 (segment (start 141 72) (end 141 90) (width 0.2) (layer "B.Cu") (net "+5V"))
 (segment (start 146.300002 74.794316) (end 143.794316 74.794316) (width 0.2) (layer "B.Cu") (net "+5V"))
 (segment (start 142.5 59.5) (end 141 59.5) (width 0.2) (layer "B.Cu") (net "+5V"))
 (segment (start 141 128.5) (end 141 130.5) (width 0.2) (layer "B.Cu") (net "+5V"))
 (segment (start 143.794316 133.294316) (end 141 130.5) (width 0.2) (layer "B.Cu") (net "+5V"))
 (segment (start 141 59.5) (end 141 71.5) (width 0.2) (layer "B.Cu") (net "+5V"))
 (segment (start 146.800002 133.294316) (end 143.794316 133.294316) (width 0.2) (layer "B.Cu") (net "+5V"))
 (segment (start 141 152) (end 141 130.5) (width 0.2) (layer "B.Cu") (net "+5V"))
 (segment (start 144 57.5) (end 144 58) (width 0.2) (layer "B.Cu") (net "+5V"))
 (segment (start 141 90) (end 141 90.5) (width 0.2) (layer "B.Cu") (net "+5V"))
 (segment (start 141 71.5) (end 141 72) (width 0.2) (layer "B.Cu") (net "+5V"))
 (segment (start 143.794316 74.794316) (end 141 72) (width 0.2) (layer "B.Cu") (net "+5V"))
 (segment (start 141 90.5) (end 141 109) (width 0.2) (layer "B.Cu") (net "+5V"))
 (segment (start 146.800002 113.794316) (end 145.794316 113.794316) (width 0.2) (layer "B.Cu") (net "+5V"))
 (segment (start 145.794316 113.794316) (end 141 109) (width 0.2) (layer "B.Cu") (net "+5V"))
 (segment (start 146.300002 94.294316) (end 144.794316 94.294316) (width 0.2) (layer "B.Cu") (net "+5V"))
 (segment (start 144.794316 94.294316) (end 141 90.5) (width 0.2) (layer "B.Cu") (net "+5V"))
 (segment (start 146.300002 76.294316) (end 146.300002 80.800002) (width 0.2) (layer "B.Cu") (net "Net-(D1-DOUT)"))
 (segment (start 146.300002 80.800002) (end 152 86.5) (width 0.2) (layer "B.Cu") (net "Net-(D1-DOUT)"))
 (segment (start 152 86.5) (end 152 93.794318) (width 0.2) (layer "B.Cu") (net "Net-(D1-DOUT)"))
 (segment (start 152 93.794318) (end 151.500002 94.294316) (width 0.2) (layer "B.Cu") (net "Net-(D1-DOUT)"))
 (segment (start 151.500002 95.794316) (end 154.794316 95.794316) (width 0.2) (layer "B.Cu") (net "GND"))
 (segment (start 152.000002 155.499998) (end 151.6 155.9) (width 0.2) (layer "B.Cu") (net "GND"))
 (segment (start 155.294316 134.794316) (end 156.5 136) (width 0.2) (layer "B.Cu") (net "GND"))
 (segment (start 140 154) (end 140 59.89896) (width 0.2) (layer "B.Cu") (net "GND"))
 (segment (start 156.5 116.5) (end 156.5 97.5) (width 0.2) (layer "B.Cu") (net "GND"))
 (segment (start 142.39896 57.5) (end 143 57.5) (width 0.2) (layer "B.Cu") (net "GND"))
 (segment (start 140 59.89896) (end 142.39896 57.5) (width 0.2) (layer "B.Cu") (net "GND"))
 (segment (start 155.294316 115.294316) (end 156.5 116.5) (width 0.2) (layer "B.Cu") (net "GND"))
 (segment (start 152.000002 154.294316) (end 155.705684 154.294316) (width 0.2) (layer "B.Cu") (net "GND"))
 (segment (start 156.5 97.5) (end 156.5 77.5) (width 0.2) (layer "B.Cu") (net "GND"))
 (segment (start 152.000002 154.294316) (end 152.000002 155.499998) (width 0.2) (layer "B.Cu") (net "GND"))
 (segment (start 152.000002 115.294316) (end 155.294316 115.294316) (width 0.2) (layer "B.Cu") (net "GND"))
 (segment (start 155.705684 154.294316) (end 156.5 153.5) (width 0.2) (layer "B.Cu") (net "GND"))
 (segment (start 156.5 77.5) (end 155.294316 76.294316) (width 0.2) (layer "B.Cu") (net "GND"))
 (segment (start 155.294316 76.294316) (end 151.500002 76.294316) (width 0.2) (layer "B.Cu") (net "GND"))
 (segment (start 154.794316 95.794316) (end 156.5 97.5) (width 0.2) (layer "B.Cu") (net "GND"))
 (segment (start 151.6 155.9) (end 141.9 155.9) (width 0.2) (layer "B.Cu") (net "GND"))
 (segment (start 152.000002 134.794316) (end 155.294316 134.794316) (width 0.2) (layer "B.Cu") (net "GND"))
 (segment (start 156.5 153.5) (end 156.5 136) (width 0.2) (layer "B.Cu") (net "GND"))
 (segment (start 141.9 155.9) (end 140 154) (width 0.2) (layer "B.Cu") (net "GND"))
 (segment (start 156.5 136) (end 156.5 116.5) (width 0.2) (layer "B.Cu") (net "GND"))
 (segment (start 147 65) (end 150 65) (width 0.2) (layer "B.Cu") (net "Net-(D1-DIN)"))
 (segment (start 150 65) (end 152.5 67.5) (width 0.2) (layer "B.Cu") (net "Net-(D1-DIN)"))
 (segment (start 145 63) (end 147 65) (width 0.2) (layer "B.Cu") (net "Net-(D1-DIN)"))
 (segment (start 152.5 67.5) (end 152.5 73.794318) (width 0.2) (layer "B.Cu") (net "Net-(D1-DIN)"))
 (segment (start 152.5 73.794318) (end 151.500002 74.794316) (width 0.2) (layer "B.Cu") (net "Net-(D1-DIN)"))
 (segment (start 145 57.5) (end 145 63) (width 0.2) (layer "B.Cu") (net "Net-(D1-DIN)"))
 (segment (start 152.000002 105.500002) (end 146.300002 99.800002) (width 0.2) (layer "B.Cu") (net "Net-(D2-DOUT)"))
 (segment (start 152.000002 113.794316) (end 152.000002 105.500002) (width 0.2) (layer "B.Cu") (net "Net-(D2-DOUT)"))
 (segment (start 146.300002 99.800002) (end 146.300002 95.794316) (width 0.2) (layer "B.Cu") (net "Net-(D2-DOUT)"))
 (segment (start 146 57) (end 146 57.5) (width 0.2) (layer "F.Cu") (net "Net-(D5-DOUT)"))
 (segment (start 141.1 152.46) (end 141.1 57.4) (width 0.2) (layer "F.Cu") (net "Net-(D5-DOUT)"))
 (segment (start 142 56.5) (end 145.5 56.5) (width 0.2) (layer "F.Cu") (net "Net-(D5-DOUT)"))
 (segment (start 145.5 56.5) (end 146 57) (width 0.2) (layer "F.Cu") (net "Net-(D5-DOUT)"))
 (segment (start 141.1 57.4) (end 142 56.5) (width 0.2) (layer "F.Cu") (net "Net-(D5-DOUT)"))
 (segment (start 143.165 154.525) (end 141.1 152.46) (width 0.2) (layer "F.Cu") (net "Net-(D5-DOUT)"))
 (segment (start 143.165 154.525) (end 146.569318 154.525) (width 0.2) (layer "B.Cu") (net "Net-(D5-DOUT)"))
 (segment (start 146.569318 154.525) (end 146.800002 154.294316) (width 0.2) (layer "B.Cu") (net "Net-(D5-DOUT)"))
 (segment (start 146.57 134.41) (end 146.57 58.505305) (width 0.2) (layer "F.Cu") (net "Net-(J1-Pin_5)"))
 (segment (start 151.58 139.42) (end 146.57 134.41) (width 0.2) (layer "F.Cu") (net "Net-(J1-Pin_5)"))
 (segment (start 151.58 139.42) (end 151.58 141.42) (width 0.2) (layer "F.Cu") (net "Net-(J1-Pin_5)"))
 (segment (start 147 58.075305) (end 147 57.5) (width 0.2) (layer "F.Cu") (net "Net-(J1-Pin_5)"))
 (segment (start 146.57 58.505305) (end 147 58.075305) (width 0.2) (layer "F.Cu") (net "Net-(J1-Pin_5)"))
 (segment (start 146.800002 139.800002) (end 146.800002 134.794316) (width 0.2) (layer "B.Cu") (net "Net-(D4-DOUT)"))
 (segment (start 152.000002 152.794316) (end 152.000002 145.000002) (width 0.2) (layer "B.Cu") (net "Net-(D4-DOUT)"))
 (segment (start 152.000002 145.000002) (end 146.800002 139.800002) (width 0.2) (layer "B.Cu") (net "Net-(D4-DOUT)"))
 (segment (start 151 57.5) (end 151 62.92) (width 0.2) (layer "F.Cu") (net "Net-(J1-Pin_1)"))
 (segment (start 151 62.92) (end 151.5 63.42) (width 0.2) (layer "F.Cu") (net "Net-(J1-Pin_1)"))
 (segment (start 152 105.5) (end 149 102.5) (width 0.2) (layer "F.Cu") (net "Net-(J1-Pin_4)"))
 (segment (start 151.5 121.92) (end 152 121.42) (width 0.2) (layer "F.Cu") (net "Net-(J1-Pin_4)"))
 (segment (start 152 98.5) (end 152 86.5) (width 0.2) (layer "F.Cu") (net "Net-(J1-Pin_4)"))
 (segment (start 152 121.42) (end 152 105.5) (width 0.2) (layer "F.Cu") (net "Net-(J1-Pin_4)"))
 (segment (start 152 86.5) (end 151.5 86) (width 0.2) (layer "F.Cu") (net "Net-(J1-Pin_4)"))
 (segment (start 151 86) (end 149.5 84.5) (width 0.2) (layer "F.Cu") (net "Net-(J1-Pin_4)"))
 (segment (start 149.5 81.5) (end 150 81) (width 0.2) (layer "F.Cu") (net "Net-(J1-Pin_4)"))
 (segment (start 151.5 86) (end 151 86) (width 0.2) (layer "F.Cu") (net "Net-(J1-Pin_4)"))
 (segment (start 149 101.5) (end 152 98.5) (width 0.2) (layer "F.Cu") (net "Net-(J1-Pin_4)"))
 (segment (start 148 64.5) (end 148 57.5) (width 0.2) (layer "F.Cu") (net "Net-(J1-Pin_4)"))
 (segment (start 149 102.5) (end 149 101.5) (width 0.2) (layer "F.Cu") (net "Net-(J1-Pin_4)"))
 (segment (start 151.5 67) (end 149 64.5) (width 0.2) (layer "F.Cu") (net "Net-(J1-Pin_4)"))
 (segment (start 150.599899 81) (end 151.5 80.099899) (width 0.2) (layer "F.Cu") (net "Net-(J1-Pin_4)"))
 (segment (start 150 81) (end 150.599899 81) (width 0.2) (layer "F.Cu") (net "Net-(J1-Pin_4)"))
 (segment (start 149.5 84.5) (end 149.5 81.5) (width 0.2) (layer "F.Cu") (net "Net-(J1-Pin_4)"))
 (segment (start 151.5 80.099899) (end 151.5 67) (width 0.2) (layer "F.Cu") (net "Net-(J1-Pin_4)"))
 (segment (start 149 64.5) (end 148 64.5) (width 0.2) (layer "F.Cu") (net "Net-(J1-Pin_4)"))
 (segment (start 148 57.5) (end 148 57.474695) (width 0.2) (layer "B.Cu") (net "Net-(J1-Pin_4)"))
 (segment (start 152.000002 133.294316) (end 152.000002 125.000002) (width 0.2) (layer "B.Cu") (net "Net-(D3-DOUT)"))
 (segment (start 146.800002 119.800002) (end 146.800002 115.294316) (width 0.2) (layer "B.Cu") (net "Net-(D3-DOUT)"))
 (segment (start 152.000002 125.000002) (end 146.800002 119.800002) (width 0.2) (layer "B.Cu") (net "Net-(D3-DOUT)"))
 (segment (start 150 59) (end 149.5 59.5) (width 0.2) (layer "F.Cu") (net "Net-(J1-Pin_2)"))
 (segment (start 151.46 82.92) (end 151.46 82.04) (width 0.2) (layer "F.Cu") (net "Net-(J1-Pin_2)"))
 (segment (start 152 66.5) (end 151.96 66.54) (width 0.2) (layer "F.Cu") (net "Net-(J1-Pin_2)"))
 (segment (start 150 57.5) (end 150 59) (width 0.2) (layer "F.Cu") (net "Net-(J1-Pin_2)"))
 (segment (start 149.5 64) (end 152 66.5) (width 0.2) (layer "F.Cu") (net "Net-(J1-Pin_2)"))
 (segment (start 149.5 59.5) (end 149.5 64) (width 0.2) (layer "F.Cu") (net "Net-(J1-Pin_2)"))
 (segment (start 151.96 66.54) (end 151.96 81.96) (width 0.2) (layer "F.Cu") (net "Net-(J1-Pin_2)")))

